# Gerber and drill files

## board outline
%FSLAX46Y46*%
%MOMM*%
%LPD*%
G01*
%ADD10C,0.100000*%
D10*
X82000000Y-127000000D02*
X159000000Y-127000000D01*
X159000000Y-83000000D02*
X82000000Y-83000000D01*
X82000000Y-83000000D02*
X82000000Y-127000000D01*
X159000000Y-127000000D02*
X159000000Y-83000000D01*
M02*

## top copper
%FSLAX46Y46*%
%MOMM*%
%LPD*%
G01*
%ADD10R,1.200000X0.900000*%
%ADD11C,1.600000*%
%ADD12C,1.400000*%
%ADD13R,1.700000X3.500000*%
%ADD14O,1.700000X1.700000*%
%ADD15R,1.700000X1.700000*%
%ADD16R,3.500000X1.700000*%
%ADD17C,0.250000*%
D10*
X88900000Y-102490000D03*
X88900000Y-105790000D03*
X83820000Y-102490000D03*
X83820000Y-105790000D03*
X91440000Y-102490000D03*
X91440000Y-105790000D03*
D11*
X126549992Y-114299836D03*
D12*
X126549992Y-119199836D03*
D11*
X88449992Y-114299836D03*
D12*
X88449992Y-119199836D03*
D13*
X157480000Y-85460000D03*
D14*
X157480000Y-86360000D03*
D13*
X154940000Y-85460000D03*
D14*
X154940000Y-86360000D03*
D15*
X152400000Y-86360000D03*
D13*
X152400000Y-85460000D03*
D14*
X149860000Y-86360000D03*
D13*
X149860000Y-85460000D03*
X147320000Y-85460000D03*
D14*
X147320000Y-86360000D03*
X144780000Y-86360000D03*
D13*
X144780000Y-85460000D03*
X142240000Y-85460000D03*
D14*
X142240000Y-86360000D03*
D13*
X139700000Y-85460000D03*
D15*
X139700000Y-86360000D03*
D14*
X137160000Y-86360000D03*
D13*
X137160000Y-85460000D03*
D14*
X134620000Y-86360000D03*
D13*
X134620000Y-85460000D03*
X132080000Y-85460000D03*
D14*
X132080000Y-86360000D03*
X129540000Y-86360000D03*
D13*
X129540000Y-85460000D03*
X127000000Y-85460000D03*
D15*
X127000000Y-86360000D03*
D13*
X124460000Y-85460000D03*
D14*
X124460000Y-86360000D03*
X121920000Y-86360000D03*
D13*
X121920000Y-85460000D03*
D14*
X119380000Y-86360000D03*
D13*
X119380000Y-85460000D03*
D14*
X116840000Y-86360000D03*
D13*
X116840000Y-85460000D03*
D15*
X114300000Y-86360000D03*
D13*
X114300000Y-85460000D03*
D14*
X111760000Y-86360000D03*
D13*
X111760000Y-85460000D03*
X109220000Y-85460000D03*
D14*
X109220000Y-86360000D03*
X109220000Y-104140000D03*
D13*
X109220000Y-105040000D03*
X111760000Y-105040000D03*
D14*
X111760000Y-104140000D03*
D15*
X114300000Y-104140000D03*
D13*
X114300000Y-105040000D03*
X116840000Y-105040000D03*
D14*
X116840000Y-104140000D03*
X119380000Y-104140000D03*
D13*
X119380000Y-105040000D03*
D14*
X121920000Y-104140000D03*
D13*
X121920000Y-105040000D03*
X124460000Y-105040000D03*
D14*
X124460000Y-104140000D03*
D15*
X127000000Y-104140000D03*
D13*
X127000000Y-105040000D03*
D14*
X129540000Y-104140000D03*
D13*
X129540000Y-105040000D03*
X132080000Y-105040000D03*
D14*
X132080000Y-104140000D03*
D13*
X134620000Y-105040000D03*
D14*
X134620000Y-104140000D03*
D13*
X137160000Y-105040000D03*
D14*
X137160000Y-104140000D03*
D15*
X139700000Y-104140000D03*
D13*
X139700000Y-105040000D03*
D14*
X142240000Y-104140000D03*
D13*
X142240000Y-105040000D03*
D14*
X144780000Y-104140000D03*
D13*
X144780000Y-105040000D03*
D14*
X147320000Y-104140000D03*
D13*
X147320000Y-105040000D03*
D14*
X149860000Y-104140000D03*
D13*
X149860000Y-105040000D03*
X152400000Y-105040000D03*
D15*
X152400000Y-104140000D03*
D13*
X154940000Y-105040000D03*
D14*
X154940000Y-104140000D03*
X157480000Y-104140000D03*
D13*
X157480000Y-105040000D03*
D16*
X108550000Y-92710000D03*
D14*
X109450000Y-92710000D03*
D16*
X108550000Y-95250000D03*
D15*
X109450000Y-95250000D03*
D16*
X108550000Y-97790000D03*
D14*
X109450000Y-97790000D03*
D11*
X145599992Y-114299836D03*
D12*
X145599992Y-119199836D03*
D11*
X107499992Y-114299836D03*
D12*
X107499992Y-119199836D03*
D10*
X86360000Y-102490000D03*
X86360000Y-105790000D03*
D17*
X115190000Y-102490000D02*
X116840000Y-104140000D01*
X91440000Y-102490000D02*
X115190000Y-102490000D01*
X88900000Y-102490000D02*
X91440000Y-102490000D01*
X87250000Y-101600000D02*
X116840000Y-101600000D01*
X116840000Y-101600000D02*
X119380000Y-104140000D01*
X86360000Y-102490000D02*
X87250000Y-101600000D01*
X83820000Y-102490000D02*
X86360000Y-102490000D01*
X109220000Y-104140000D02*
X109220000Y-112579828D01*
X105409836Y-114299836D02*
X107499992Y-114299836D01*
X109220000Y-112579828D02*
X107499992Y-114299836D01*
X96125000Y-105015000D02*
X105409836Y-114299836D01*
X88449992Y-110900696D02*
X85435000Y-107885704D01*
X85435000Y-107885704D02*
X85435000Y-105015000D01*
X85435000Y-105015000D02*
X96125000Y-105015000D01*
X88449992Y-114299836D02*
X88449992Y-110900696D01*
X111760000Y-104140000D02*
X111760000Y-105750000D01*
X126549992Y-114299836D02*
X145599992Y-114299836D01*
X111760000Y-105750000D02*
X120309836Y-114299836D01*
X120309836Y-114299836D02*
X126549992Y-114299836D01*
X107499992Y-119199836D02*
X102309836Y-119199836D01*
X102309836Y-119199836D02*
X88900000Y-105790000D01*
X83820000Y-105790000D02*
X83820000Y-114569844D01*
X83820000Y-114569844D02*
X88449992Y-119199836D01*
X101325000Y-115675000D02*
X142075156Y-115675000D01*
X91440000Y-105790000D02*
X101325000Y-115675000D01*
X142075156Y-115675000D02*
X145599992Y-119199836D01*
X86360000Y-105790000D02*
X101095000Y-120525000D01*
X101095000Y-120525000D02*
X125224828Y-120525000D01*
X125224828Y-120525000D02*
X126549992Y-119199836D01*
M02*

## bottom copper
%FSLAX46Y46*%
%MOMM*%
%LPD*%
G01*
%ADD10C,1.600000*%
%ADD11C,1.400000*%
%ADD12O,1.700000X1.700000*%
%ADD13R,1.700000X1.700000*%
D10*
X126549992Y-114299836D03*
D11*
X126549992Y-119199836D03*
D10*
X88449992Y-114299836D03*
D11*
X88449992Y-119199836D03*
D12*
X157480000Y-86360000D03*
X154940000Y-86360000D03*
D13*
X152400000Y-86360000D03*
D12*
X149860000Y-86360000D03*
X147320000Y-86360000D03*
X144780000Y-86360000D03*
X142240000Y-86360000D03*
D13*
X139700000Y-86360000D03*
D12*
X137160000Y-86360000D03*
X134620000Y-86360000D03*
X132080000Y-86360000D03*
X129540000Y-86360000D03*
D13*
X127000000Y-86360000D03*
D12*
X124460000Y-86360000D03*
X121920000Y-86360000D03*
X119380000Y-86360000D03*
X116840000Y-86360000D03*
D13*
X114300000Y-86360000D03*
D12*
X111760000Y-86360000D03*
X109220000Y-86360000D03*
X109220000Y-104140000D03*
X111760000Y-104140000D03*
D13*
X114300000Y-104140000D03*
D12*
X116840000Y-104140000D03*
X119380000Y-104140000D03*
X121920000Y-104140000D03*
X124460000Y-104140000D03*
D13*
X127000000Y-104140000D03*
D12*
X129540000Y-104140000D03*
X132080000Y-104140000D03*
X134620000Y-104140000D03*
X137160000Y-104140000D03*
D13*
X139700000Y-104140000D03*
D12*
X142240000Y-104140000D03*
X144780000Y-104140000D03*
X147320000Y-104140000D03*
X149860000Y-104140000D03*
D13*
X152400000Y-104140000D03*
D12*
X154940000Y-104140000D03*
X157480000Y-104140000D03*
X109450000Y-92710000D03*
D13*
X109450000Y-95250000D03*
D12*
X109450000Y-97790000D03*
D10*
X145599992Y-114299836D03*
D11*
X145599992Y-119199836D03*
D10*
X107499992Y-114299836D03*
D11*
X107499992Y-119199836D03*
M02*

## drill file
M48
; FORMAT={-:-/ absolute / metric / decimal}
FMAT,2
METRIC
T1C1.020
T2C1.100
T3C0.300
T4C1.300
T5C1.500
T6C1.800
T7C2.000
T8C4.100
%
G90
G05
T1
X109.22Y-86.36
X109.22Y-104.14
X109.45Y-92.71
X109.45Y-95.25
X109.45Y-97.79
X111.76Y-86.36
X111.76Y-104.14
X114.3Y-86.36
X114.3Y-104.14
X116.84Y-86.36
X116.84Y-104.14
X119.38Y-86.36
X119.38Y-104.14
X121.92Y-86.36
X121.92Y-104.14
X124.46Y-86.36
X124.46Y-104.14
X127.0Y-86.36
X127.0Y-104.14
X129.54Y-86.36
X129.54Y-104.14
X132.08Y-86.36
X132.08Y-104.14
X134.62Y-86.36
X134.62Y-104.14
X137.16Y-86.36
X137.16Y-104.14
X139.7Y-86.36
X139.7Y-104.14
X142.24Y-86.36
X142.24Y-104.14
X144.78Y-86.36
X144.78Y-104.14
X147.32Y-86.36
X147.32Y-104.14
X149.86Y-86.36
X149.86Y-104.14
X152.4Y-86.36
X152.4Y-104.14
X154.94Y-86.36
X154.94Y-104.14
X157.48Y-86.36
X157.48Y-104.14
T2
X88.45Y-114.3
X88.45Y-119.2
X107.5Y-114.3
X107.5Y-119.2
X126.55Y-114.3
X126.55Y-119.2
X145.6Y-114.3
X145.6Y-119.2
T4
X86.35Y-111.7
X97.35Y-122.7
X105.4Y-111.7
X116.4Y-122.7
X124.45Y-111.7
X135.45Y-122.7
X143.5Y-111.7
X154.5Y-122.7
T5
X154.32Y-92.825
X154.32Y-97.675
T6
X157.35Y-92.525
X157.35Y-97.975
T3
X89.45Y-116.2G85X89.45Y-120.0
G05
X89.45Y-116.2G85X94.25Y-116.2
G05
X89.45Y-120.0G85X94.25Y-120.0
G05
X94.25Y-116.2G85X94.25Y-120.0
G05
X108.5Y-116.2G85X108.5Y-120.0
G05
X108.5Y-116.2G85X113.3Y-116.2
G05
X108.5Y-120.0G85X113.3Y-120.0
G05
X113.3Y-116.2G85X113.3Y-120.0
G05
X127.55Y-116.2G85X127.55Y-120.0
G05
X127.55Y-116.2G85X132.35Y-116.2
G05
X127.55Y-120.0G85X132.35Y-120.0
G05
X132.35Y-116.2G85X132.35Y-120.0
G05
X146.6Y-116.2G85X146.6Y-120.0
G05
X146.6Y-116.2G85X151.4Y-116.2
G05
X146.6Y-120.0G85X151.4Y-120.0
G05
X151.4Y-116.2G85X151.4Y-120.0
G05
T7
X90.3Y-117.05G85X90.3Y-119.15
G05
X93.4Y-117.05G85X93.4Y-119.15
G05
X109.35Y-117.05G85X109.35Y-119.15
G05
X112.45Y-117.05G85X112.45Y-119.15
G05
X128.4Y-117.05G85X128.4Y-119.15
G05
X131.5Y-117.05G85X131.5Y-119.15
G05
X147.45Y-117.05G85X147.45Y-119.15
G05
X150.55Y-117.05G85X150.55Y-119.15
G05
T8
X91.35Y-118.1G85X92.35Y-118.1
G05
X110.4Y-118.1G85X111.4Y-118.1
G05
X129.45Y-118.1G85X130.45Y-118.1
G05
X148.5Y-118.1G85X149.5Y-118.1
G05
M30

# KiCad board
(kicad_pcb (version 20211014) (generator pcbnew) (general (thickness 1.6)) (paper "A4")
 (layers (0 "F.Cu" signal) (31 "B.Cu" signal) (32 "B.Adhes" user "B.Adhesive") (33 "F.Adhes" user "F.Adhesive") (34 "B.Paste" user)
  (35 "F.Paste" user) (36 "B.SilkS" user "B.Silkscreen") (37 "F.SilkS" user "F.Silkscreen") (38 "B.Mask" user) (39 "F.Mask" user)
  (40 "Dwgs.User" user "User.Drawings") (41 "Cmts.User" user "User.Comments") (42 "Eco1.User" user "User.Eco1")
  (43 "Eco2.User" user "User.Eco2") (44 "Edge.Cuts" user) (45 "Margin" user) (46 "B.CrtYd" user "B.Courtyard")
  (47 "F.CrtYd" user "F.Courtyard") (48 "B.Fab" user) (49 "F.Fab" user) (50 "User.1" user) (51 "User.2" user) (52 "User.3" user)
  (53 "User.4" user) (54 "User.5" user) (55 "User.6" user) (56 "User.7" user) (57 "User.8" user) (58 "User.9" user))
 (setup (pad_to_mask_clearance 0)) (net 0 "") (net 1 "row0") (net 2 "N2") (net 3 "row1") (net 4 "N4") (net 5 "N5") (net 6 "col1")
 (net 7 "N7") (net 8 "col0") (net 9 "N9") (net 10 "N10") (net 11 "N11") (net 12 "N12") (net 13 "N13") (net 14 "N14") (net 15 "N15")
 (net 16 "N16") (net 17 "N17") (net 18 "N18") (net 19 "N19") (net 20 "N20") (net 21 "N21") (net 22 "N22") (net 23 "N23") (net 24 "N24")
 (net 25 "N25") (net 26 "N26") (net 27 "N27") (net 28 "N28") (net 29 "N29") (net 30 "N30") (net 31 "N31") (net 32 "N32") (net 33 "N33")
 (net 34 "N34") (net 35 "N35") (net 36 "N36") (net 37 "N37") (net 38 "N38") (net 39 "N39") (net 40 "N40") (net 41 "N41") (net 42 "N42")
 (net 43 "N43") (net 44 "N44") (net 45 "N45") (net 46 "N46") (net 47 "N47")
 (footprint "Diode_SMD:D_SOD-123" (layer "F.Cu") (at 88.9 104.14 -90)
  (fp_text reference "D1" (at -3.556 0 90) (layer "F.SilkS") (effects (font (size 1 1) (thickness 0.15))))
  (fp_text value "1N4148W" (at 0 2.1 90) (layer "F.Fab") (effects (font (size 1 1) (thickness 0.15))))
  (pad "1" smd rect (at -1.65 0 270) (size 0.9 1.2) (layers "F.Cu" "F.Paste" "F.Mask") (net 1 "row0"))
  (pad "2" smd rect (at 1.65 0 270) (size 0.9 1.2) (layers "F.Cu" "F.Paste" "F.Mask") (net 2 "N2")))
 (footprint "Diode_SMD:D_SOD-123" (layer "F.Cu") (at 83.82 104.14 -90)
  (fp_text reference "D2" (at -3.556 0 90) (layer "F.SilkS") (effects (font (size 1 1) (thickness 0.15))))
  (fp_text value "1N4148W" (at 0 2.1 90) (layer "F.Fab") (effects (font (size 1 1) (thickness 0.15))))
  (pad "1" smd rect (at -1.65 0 270) (size 0.9 1.2) (layers "F.Cu" "F.Paste" "F.Mask") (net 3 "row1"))
  (pad "2" smd rect (at 1.65 0 270) (size 0.9 1.2) (layers "F.Cu" "F.Paste" "F.Mask") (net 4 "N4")))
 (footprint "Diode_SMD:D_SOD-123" (layer "F.Cu") (at 91.44 104.14 -90)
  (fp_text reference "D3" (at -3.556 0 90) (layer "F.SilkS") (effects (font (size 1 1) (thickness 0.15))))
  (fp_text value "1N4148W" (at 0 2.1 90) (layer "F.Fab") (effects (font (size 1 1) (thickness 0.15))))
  (pad "1" smd rect (at -1.65 0 270) (size 0.9 1.2) (layers "F.Cu" "F.Paste" "F.Mask") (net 1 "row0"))
  (pad "2" smd rect (at 1.65 0 270) (size 0.9 1.2) (layers "F.Cu" "F.Paste" "F.Mask") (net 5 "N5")))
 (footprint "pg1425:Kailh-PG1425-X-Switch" (layer "F.Cu") (at 133.35 114.3)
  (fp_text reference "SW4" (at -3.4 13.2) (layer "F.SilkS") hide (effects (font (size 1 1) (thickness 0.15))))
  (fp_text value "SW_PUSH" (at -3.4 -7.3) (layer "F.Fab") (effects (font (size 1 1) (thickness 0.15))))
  (pad "" np_thru_hole oval locked (at -3.4 3.8) (size 5.1 4.1) (drill oval 5.1 4.1) (layers *.Cu *.Mask))
  (pad "" np_thru_hole oval locked (at -1.85 3.8) (size 2 4.1) (drill oval 2 4.1) (layers *.Cu *.Mask))
  (pad "" np_thru_hole oval locked (at -5.8 3.8) (size 0.3 4.1) (drill oval 0.3 4.1) (layers *.Cu *.Mask))
  (pad "" np_thru_hole oval locked (at -3.4 1.9) (size 5.1 0.3) (drill oval 5.1 0.3) (layers *.Cu *.Mask))
  (pad "" np_thru_hole circle locked (at -8.900008 -2.600164 180) (size 1.3 1.3) (drill 1.3) (layers *.Cu *.Mask))
  (pad "" np_thru_hole oval locked (at -3.4 5.7) (size 5.1 0.3) (drill oval 5.1 0.3) (layers *.Cu *.Mask))
  (pad "" np_thru_hole oval locked (at -4.95 3.8) (size 2 4.1) (drill oval 2 4.1) (layers *.Cu *.Mask))
  (pad "" np_thru_hole oval locked (at -1 3.8) (size 0.3 4.1) (drill oval 0.3 4.1) (layers *.Cu *.Mask))
  (pad "" np_thru_hole circle locked (at 2.099992 8.399836 180) (size 1.3 1.3) (drill 1.3) (layers *.Cu *.Mask))
  (pad "1" thru_hole circle locked (at -6.800008 -0.000164 180) (size 1.6 1.6) (drill 1.1) (layers *.Cu *.Mask) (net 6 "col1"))
  (pad "2" thru_hole circle locked (at -6.800008 4.899836 180) (size 1.4 1.4) (drill 1.1) (layers *.Cu *.Mask) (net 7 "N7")))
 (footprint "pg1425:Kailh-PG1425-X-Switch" (layer "F.Cu") (at 95.25 114.3)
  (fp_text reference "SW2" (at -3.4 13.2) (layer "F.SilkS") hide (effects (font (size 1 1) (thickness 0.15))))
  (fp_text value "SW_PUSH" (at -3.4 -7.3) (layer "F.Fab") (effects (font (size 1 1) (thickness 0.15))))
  (pad "" np_thru_hole oval locked (at -4.95 3.8) (size 2 4.1) (drill oval 2 4.1) (layers *.Cu *.Mask))
  (pad "" np_thru_hole oval locked (at -5.8 3.8) (size 0.3 4.1) (drill oval 0.3 4.1) (layers *.Cu *.Mask))
  (pad "" np_thru_hole oval locked (at -1 3.8) (size 0.3 4.1) (drill oval 0.3 4.1) (layers *.Cu *.Mask))
  (pad "" np_thru_hole oval locked (at -1.85 3.8) (size 2 4.1) (drill oval 2 4.1) (layers *.Cu *.Mask))
  (pad "" np_thru_hole circle locked (at -8.900008 -2.600164 180) (size 1.3 1.3) (drill 1.3) (layers *.Cu *.Mask))
  (pad "" np_thru_hole oval locked (at -3.4 3.8) (size 5.1 4.1) (drill oval 5.1 4.1) (layers *.Cu *.Mask))
  (pad "" np_thru_hole oval locked (at -3.4 5.7) (size 5.1 0.3) (drill oval 5.1 0.3) (layers *.Cu *.Mask))
  (pad "" np_thru_hole oval locked (at -3.4 1.9) (size 5.1 0.3) (drill oval 5.1 0.3) (layers *.Cu *.Mask))
  (pad "" np_thru_hole circle locked (at 2.099992 8.399836 180) (size 1.3 1.3) (drill 1.3) (layers *.Cu *.Mask))
  (pad "1" thru_hole circle locked (at -6.800008 -0.000164 180) (size 1.6 1.6) (drill 1.1) (layers *.Cu *.Mask) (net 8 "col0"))
  (pad "2" thru_hole circle locked (at -6.800008 4.899836 180) (size 1.4 1.4) (drill 1.1) (layers *.Cu *.Mask) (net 4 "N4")))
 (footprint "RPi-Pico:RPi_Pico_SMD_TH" (layer "F.Cu") (at 133.35 95.25 -90)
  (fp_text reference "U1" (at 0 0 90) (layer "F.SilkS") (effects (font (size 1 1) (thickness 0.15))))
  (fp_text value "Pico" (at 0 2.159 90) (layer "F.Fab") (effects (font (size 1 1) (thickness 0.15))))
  (pad "" np_thru_hole oval (at 2.725 -24 270) (size 1.8 1.8) (drill 1.8) (layers *.Cu *.Mask))
  (pad "" np_thru_hole oval (at -2.425 -20.97 270) (size 1.5 1.5) (drill 1.5) (layers *.Cu *.Mask))
  (pad "" np_thru_hole oval (at -2.725 -24 270) (size 1.8 1.8) (drill 1.8) (layers *.Cu *.Mask))
  (pad "" np_thru_hole oval (at 2.425 -20.97 270) (size 1.5 1.5) (drill 1.5) (layers *.Cu *.Mask))
  (pad "1" smd rect (at -8.89 -24.13 270) (size 3.5 1.7) (drill (offset -0.9 0)) (layers "F.Cu" "F.Mask") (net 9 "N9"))
  (pad "1" thru_hole oval (at -8.89 -24.13 270) (size 1.7 1.7) (drill 1.02) (layers *.Cu *.Mask) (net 9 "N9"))
  (pad "2" smd rect (at -8.89 -21.59 270) (size 3.5 1.7) (drill (offset -0.9 0)) (layers "F.Cu" "F.Mask") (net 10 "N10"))
  (pad "2" thru_hole oval (at -8.89 -21.59 270) (size 1.7 1.7) (drill 1.02) (layers *.Cu *.Mask) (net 10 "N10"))
  (pad "3" thru_hole rect (at -8.89 -19.05 270) (size 1.7 1.7) (drill 1.02) (layers *.Cu *.Mask) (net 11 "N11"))
  (pad "3" smd rect (at -8.89 -19.05 270) (size 3.5 1.7) (drill (offset -0.9 0)) (layers "F.Cu" "F.Mask") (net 11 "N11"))
  (pad "4" thru_hole oval (at -8.89 -16.51 270) (size 1.7 1.7) (drill 1.02) (layers *.Cu *.Mask) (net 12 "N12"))
  (pad "4" smd rect (at -8.89 -16.51 270) (size 3.5 1.7) (drill (offset -0.9 0)) (layers "F.Cu" "F.Mask") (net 12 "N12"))
  (pad "5" smd rect (at -8.89 -13.97 270) (size 3.5 1.7) (drill (offset -0.9 0)) (layers "F.Cu" "F.Mask") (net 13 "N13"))
  (pad "5" thru_hole oval (at -8.89 -13.97 270) (size 1.7 1.7) (drill 1.02) (layers *.Cu *.Mask) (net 13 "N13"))
  (pad "6" thru_hole oval (at -8.89 -11.43 270) (size 1.7 1.7) (drill 1.02) (layers *.Cu *.Mask) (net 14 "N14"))
  (pad "6" smd rect (at -8.89 -11.43 270) (size 3.5 1.7) (drill (offset -0.9 0)) (layers "F.Cu" "F.Mask") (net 14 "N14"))
  (pad "7" smd rect (at -8.89 -8.89 270) (size 3.5 1.7) (drill (offset -0.9 0)) (layers "F.Cu" "F.Mask") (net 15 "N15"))
  (pad "7" thru_hole oval (at -8.89 -8.89 270) (size 1.7 1.7) (drill 1.02) (layers *.Cu *.Mask) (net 15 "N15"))
  (pad "8" smd rect (at -8.89 -6.35 270) (size 3.5 1.7) (drill (offset -0.9 0)) (layers "F.Cu" "F.Mask") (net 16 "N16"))
  (pad "8" thru_hole rect (at -8.89 -6.35 270) (size 1.7 1.7) (drill 1.02) (layers *.Cu *.Mask) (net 16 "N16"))
  (pad "9" thru_hole oval (at -8.89 -3.81 270) (size 1.7 1.7) (drill 1.02) (layers *.Cu *.Mask) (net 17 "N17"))
  (pad "9" smd rect (at -8.89 -3.81 270) (size 3.5 1.7) (drill (offset -0.9 0)) (layers "F.Cu" "F.Mask") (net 17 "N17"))
  (pad "10" thru_hole oval (at -8.89 -1.27 270) (size 1.7 1.7) (drill 1.02) (layers *.Cu *.Mask) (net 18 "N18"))
  (pad "10" smd rect (at -8.89 -1.27 270) (size 3.5 1.7) (drill (offset -0.9 0)) (layers "F.Cu" "F.Mask") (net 18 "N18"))
  (pad "11" smd rect (at -8.89 1.27 270) (size 3.5 1.7) (drill (offset -0.9 0)) (layers "F.Cu" "F.Mask") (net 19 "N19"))
  (pad "11" thru_hole oval (at -8.89 1.27 270) (size 1.7 1.7) (drill 1.02) (layers *.Cu *.Mask) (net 19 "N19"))
  (pad "12" thru_hole oval (at -8.89 3.81 270) (size 1.7 1.7) (drill 1.02) (layers *.Cu *.Mask) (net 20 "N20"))
  (pad "12" smd rect (at -8.89 3.81 270) (size 3.5 1.7) (drill (offset -0.9 0)) (layers "F.Cu" "F.Mask") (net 20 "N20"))
  (pad "13" smd rect (at -8.89 6.35 270) (size 3.5 1.7) (drill (offset -0.9 0)) (layers "F.Cu" "F.Mask") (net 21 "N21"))
  (pad "13" thru_hole rect (at -8.89 6.35 270) (size 1.7 1.7) (drill 1.02) (layers *.Cu *.Mask) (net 21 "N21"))
  (pad "14" smd rect (at -8.89 8.89 270) (size 3.5 1.7) (drill (offset -0.9 0)) (layers "F.Cu" "F.Mask") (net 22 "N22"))
  (pad "14" thru_hole oval (at -8.89 8.89 270) (size 1.7 1.7) (drill 1.02) (layers *.Cu *.Mask) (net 22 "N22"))
  (pad "15" thru_hole oval (at -8.89 11.43 270) (size 1.7 1.7) (drill 1.02) (layers *.Cu *.Mask) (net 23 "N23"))
  (pad "15" smd rect (at -8.89 11.43 270) (size 3.5 1.7) (drill (offset -0.9 0)) (layers "F.Cu" "F.Mask") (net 23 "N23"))
  (pad "16" thru_hole oval (at -8.89 13.97 270) (size 1.7 1.7) (drill 1.02) (layers *.Cu *.Mask) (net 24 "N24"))
  (pad "16" smd rect (at -8.89 13.97 270) (size 3.5 1.7) (drill (offset -0.9 0)) (layers "F.Cu" "F.Mask") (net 24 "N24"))
  (pad "17" thru_hole oval (at -8.89 16.51 270) (size 1.7 1.7) (drill 1.02) (layers *.Cu *.Mask) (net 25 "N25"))
  (pad "17" smd rect (at -8.89 16.51 270) (size 3.5 1.7) (drill (offset -0.9 0)) (layers "F.Cu" "F.Mask") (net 25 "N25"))
  (pad "18" thru_hole rect (at -8.89 19.05 270) (size 1.7 1.7) (drill 1.02) (layers *.Cu *.Mask) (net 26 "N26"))
  (pad "18" smd rect (at -8.89 19.05 270) (size 3.5 1.7) (drill (offset -0.9 0)) (layers "F.Cu" "F.Mask") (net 26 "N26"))
  (pad "19" thru_hole oval (at -8.89 21.59 270) (size 1.7 1.7) (drill 1.02) (layers *.Cu *.Mask) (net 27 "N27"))
  (pad "19" smd rect (at -8.89 21.59 270) (size 3.5 1.7) (drill (offset -0.9 0)) (layers "F.Cu" "F.Mask") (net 27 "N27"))
  (pad "20" smd rect (at -8.89 24.13 270) (size 3.5 1.7) (drill (offset -0.9 0)) (layers "F.Cu" "F.Mask") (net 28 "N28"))
  (pad "20" thru_hole oval (at -8.89 24.13 270) (size 1.7 1.7) (drill 1.02) (layers *.Cu *.Mask) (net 28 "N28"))
  (pad "21" thru_hole oval (at 8.89 24.13 270) (size 1.7 1.7) (drill 1.02) (layers *.Cu *.Mask) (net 8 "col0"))
  (pad "21" smd rect (at 8.89 24.13 270) (size 3.5 1.7) (drill (offset 0.9 0)) (layers "F.Cu" "F.Mask") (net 8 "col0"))
  (pad "22" smd rect (at 8.89 21.59 270) (size 3.5 1.7) (drill (offset 0.9 0)) (layers "F.Cu" "F.Mask") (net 6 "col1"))
  (pad "22" thru_hole oval (at 8.89 21.59 270) (size 1.7 1.7) (drill 1.02) (layers *.Cu *.Mask) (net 6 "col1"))
  (pad "23" thru_hole rect (at 8.89 19.05 270) (size 1.7 1.7) (drill 1.02) (layers *.Cu *.Mask) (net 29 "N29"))
  (pad "23" smd rect (at 8.89 19.05 270) (size 3.5 1.7) (drill (offset 0.9 0)) (layers "F.Cu" "F.Mask") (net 29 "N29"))
  (pad "24" smd rect (at 8.89 16.51 270) (size 3.5 1.7) (drill (offset 0.9 0)) (layers "F.Cu" "F.Mask") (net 1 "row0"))
  (pad "24" thru_hole oval (at 8.89 16.51 270) (size 1.7 1.7) (drill 1.02) (layers *.Cu *.Mask) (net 1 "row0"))
  (pad "25" thru_hole oval (at 8.89 13.97 270) (size 1.7 1.7) (drill 1.02) (layers *.Cu *.Mask) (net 3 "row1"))
  (pad "25" smd rect (at 8.89 13.97 270) (size 3.5 1.7) (drill (offset 0.9 0)) (layers "F.Cu" "F.Mask") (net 3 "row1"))
  (pad "26" thru_hole oval (at 8.89 11.43 270) (size 1.7 1.7) (drill 1.02) (layers *.Cu *.Mask) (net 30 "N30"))
  (pad "26" smd rect (at 8.89 11.43 270) (size 3.5 1.7) (drill (offset 0.9 0)) (layers "F.Cu" "F.Mask") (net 30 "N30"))
  (pad "27" smd rect (at 8.89 8.89 270) (size 3.5 1.7) (drill (offset 0.9 0)) (layers "F.Cu" "F.Mask") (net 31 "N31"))
  (pad "27" thru_hole oval (at 8.89 8.89 270) (size 1.7 1.7) (drill 1.02) (layers *.Cu *.Mask) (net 31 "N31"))
  (pad "28" thru_hole rect (at 8.89 6.35 270) (size 1.7 1.7) (drill 1.02) (layers *.Cu *.Mask) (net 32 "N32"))
  (pad "28" smd rect (at 8.89 6.35 270) (size 3.5 1.7) (drill (offset 0.9 0)) (layers "F.Cu" "F.Mask") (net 32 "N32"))
  (pad "29" thru_hole oval (at 8.89 3.81 270) (size 1.7 1.7) (drill 1.02) (layers *.Cu *.Mask) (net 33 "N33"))
  (pad "29" smd rect (at 8.89 3.81 270) (size 3.5 1.7) (drill (offset 0.9 0)) (layers "F.Cu" "F.Mask") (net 33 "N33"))
  (pad "30" smd rect (at 8.89 1.27 270) (size 3.5 1.7) (drill (offset 0.9 0)) (layers "F.Cu" "F.Mask") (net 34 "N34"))
  (pad "30" thru_hole oval (at 8.89 1.27 270) (size 1.7 1.7) (drill 1.02) (layers *.Cu *.Mask) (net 34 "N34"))
  (pad "31" smd rect (at 8.89 -1.27 270) (size 3.5 1.7) (drill (offset 0.9 0)) (layers "F.Cu" "F.Mask") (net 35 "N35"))
  (pad "31" thru_hole oval (at 8.89 -1.27 270) (size 1.7 1.7) (drill 1.02) (layers *.Cu *.Mask) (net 35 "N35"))
  (pad "32" smd rect (at 8.89 -3.81 270) (size 3.5 1.7) (drill (offset 0.9 0)) (layers "F.Cu" "F.Mask") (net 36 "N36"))
  (pad "32" thru_hole oval (at 8.89 -3.81 270) (size 1.7 1.7) (drill 1.02) (layers *.Cu *.Mask) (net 36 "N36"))
  (pad "33" thru_hole rect (at 8.89 -6.35 270) (size 1.7 1.7) (drill 1.02) (layers *.Cu *.Mask) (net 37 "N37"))
  (pad "33" smd rect (at 8.89 -6.35 270) (size 3.5 1.7) (drill (offset 0.9 0)) (layers "F.Cu" "F.Mask") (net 37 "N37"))
  (pad "34" thru_hole oval (at 8.89 -8.89 270) (size 1.7 1.7) (drill 1.02) (layers *.Cu *.Mask) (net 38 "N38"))
  (pad "34" smd rect (at 8.89 -8.89 270) (size 3.5 1.7) (drill (offset 0.9 0)) (layers "F.Cu" "F.Mask") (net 38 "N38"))
  (pad "35" thru_hole oval (at 8.89 -11.43 270) (size 1.7 1.7) (drill 1.02) (layers *.Cu *.Mask) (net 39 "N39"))
  (pad "35" smd rect (at 8.89 -11.43 270) (size 3.5 1.7) (drill (offset 0.9 0)) (layers "F.Cu" "F.Mask") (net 39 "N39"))
  (pad "36" thru_hole oval (at 8.89 -13.97 270) (size 1.7 1.7) (drill 1.02) (layers *.Cu *.Mask) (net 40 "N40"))
  (pad "36" smd rect (at 8.89 -13.97 270) (size 3.5 1.7) (drill (offset 0.9 0)) (layers "F.Cu" "F.Mask") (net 40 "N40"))
  (pad "37" thru_hole oval (at 8.89 -16.51 270) (size 1.7 1.7) (drill 1.02) (layers *.Cu *.Mask) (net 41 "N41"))
  (pad "37" smd rect (at 8.89 -16.51 270) (size 3.5 1.7) (drill (offset 0.9 0)) (layers "F.Cu" "F.Mask") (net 41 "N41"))
  (pad "38" smd rect (at 8.89 -19.05 270) (size 3.5 1.7) (drill (offset 0.9 0)) (layers "F.Cu" "F.Mask") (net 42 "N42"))
  (pad "38" thru_hole rect (at 8.89 -19.05 270) (size 1.7 1.7) (drill 1.02) (layers *.Cu *.Mask) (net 42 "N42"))
  (pad "39" smd rect (at 8.89 -21.59 270) (size 3.5 1.7) (drill (offset 0.9 0)) (layers "F.Cu" "F.Mask") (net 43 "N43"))
  (pad "39" thru_hole oval (at 8.89 -21.59 270) (size 1.7 1.7) (drill 1.02) (layers *.Cu *.Mask) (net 43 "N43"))
  (pad "40" thru_hole oval (at 8.89 -24.13 270) (size 1.7 1.7) (drill 1.02) (layers *.Cu *.Mask) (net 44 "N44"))
  (pad "40" smd rect (at 8.89 -24.13 270) (size 3.5 1.7) (drill (offset 0.9 0)) (layers "F.Cu" "F.Mask") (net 44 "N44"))
  (pad "41" smd rect (at -2.54 23.9) (size 3.5 1.7) (drill (offset -0.9 0)) (layers "F.Cu" "F.Mask") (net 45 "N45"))
  (pad "41" thru_hole oval (at -2.54 23.9 270) (size 1.7 1.7) (drill 1.02) (layers *.Cu *.Mask) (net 45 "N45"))
  (pad "42" smd rect (at 0 23.9) (size 3.5 1.7) (drill (offset -0.9 0)) (layers "F.Cu" "F.Mask") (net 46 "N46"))
  (pad "42" thru_hole rect (at 0 23.9 270) (size 1.7 1.7) (drill 1.02) (layers *.Cu *.Mask) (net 46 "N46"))
  (pad "43" smd rect (at 2.54 23.9) (size 3.5 1.7) (drill (offset -0.9 0)) (layers "F.Cu" "F.Mask") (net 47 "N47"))
  (pad "43" thru_hole oval (at 2.54 23.9 270) (size 1.7 1.7) (drill 1.02) (layers *.Cu *.Mask) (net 47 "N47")))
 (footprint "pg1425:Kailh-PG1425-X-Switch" (layer "F.Cu") (at 152.4 114.3)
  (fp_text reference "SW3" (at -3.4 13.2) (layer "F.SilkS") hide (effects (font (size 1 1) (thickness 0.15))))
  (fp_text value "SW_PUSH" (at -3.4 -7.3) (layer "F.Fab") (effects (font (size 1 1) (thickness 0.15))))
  (pad "" np_thru_hole oval locked (at -1.85 3.8) (size 2 4.1) (drill oval 2 4.1) (layers *.Cu *.Mask))
  (pad "" np_thru_hole circle locked (at 2.099992 8.399836 180) (size 1.3 1.3) (drill 1.3) (layers *.Cu *.Mask))
  (pad "" np_thru_hole circle locked (at -8.900008 -2.600164 180) (size 1.3 1.3) (drill 1.3) (layers *.Cu *.Mask))
  (pad "" np_thru_hole oval locked (at -3.4 1.9) (size 5.1 0.3) (drill oval 5.1 0.3) (layers *.Cu *.Mask))
  (pad "" np_thru_hole oval locked (at -1 3.8) (size 0.3 4.1) (drill oval 0.3 4.1) (layers *.Cu *.Mask))
  (pad "" np_thru_hole oval locked (at -3.4 3.8) (size 5.1 4.1) (drill oval 5.1 4.1) (layers *.Cu *.Mask))
  (pad "" np_thru_hole oval locked (at -3.4 5.7) (size 5.1 0.3) (drill oval 5.1 0.3) (layers *.Cu *.Mask))
  (pad "" np_thru_hole oval locked (at -5.8 3.8) (size 0.3 4.1) (drill oval 0.3 4.1) (layers *.Cu *.Mask))
  (pad "" np_thru_hole oval locked (at -4.95 3.8) (size 2 4.1) (drill oval 2 4.1) (layers *.Cu *.Mask))
  (pad "1" thru_hole circle locked (at -6.800008 -0.000164 180) (size 1.6 1.6) (drill 1.1) (layers *.Cu *.Mask) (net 6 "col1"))
  (pad "2" thru_hole circle locked (at -6.800008 4.899836 180) (size 1.4 1.4) (drill 1.1) (layers *.Cu *.Mask) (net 5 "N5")))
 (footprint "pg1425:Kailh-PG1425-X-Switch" (layer "F.Cu") (at 114.3 114.3)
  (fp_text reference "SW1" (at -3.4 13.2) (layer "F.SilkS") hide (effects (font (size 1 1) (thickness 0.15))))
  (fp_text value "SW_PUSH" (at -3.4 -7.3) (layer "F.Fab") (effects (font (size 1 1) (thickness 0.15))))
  (pad "" np_thru_hole oval locked (at -3.4 3.8) (size 5.1 4.1) (drill oval 5.1 4.1) (layers *.Cu *.Mask))
  (pad "" np_thru_hole oval locked (at -5.8 3.8) (size 0.3 4.1) (drill oval 0.3 4.1) (layers *.Cu *.Mask))
  (pad "" np_thru_hole oval locked (at -1 3.8) (size 0.3 4.1) (drill oval 0.3 4.1) (layers *.Cu *.Mask))
  (pad "" np_thru_hole circle locked (at -8.900008 -2.600164 180) (size 1.3 1.3) (drill 1.3) (layers *.Cu *.Mask))
  (pad "" np_thru_hole oval locked (at -3.4 1.9) (size 5.1 0.3) (drill oval 5.1 0.3) (layers *.Cu *.Mask))
  (pad "" np_thru_hole oval locked (at -3.4 5.7) (size 5.1 0.3) (drill oval 5.1 0.3) (layers *.Cu *.Mask))
  (pad "" np_thru_hole oval locked (at -1.85 3.8) (size 2 4.1) (drill oval 2 4.1) (layers *.Cu *.Mask))
  (pad "" np_thru_hole circle locked (at 2.099992 8.399836 180) (size 1.3 1.3) (drill 1.3) (layers *.Cu *.Mask))
  (pad "" np_thru_hole oval locked (at -4.95 3.8) (size 2 4.1) (drill oval 2 4.1) (layers *.Cu *.Mask))
  (pad "1" thru_hole circle locked (at -6.800008 -0.000164 180) (size 1.6 1.6) (drill 1.1) (layers *.Cu *.Mask) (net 8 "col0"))
  (pad "2" thru_hole circle locked (at -6.800008 4.899836 180) (size 1.4 1.4) (drill 1.1) (layers *.Cu *.Mask) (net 2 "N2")))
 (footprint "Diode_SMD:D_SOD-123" (layer "F.Cu") (at 86.36 104.14 -90)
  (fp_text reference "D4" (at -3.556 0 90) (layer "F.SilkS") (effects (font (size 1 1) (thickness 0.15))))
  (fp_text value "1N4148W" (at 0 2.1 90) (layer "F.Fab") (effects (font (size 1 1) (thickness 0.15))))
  (pad "1" smd rect (at -1.65 0 270) (size 0.9 1.2) (layers "F.Cu" "F.Paste" "F.Mask") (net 3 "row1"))
  (pad "2" smd rect (at 1.65 0 270) (size 0.9 1.2) (layers "F.Cu" "F.Paste" "F.Mask") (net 7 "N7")))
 (gr_line (start 82 127) (end 159 127) (layer "Edge.Cuts") (width 0.1))
 (gr_line (start 159 83) (end 82 83) (layer "Edge.Cuts") (width 0.1))
 (gr_line (start 82 83) (end 82 127) (layer "Edge.Cuts") (width 0.1))
 (gr_line (start 159 127) (end 159 83) (layer "Edge.Cuts") (width 0.1))
 (segment (start 115.19 102.49) (end 116.84 104.14) (width 0.25) (layer "F.Cu") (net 1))
 (segment (start 91.44 102.49) (end 115.19 102.49) (width 0.25) (layer "F.Cu") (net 1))
 (segment (start 88.9 102.49) (end 91.44 102.49) (width 0.25) (layer "F.Cu") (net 1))
 (segment (start 87.25 101.6) (end 116.84 101.6) (width 0.25) (layer "F.Cu") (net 3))
 (segment (start 116.84 101.6) (end 119.38 104.14) (width 0.25) (layer "F.Cu") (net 3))
 (segment (start 86.36 102.49) (end 87.25 101.6) (width 0.25) (layer "F.Cu") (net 3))
 (segment (start 83.82 102.49) (end 86.36 102.49) (width 0.25) (layer "F.Cu") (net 3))
 (segment (start 109.22 104.14) (end 109.22 112.579828) (width 0.25) (layer "F.Cu") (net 8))
 (segment (start 105.409836 114.299836) (end 107.499992 114.299836) (width 0.25) (layer "F.Cu") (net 8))
 (segment (start 109.22 112.579828) (end 107.499992 114.299836) (width 0.25) (layer "F.Cu") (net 8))
 (segment (start 96.125 105.015) (end 105.409836 114.299836) (width 0.25) (layer "F.Cu") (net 8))
 (segment (start 88.449992 110.900696) (end 85.435 107.885704) (width 0.25) (layer "F.Cu") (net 8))
 (segment (start 85.435 107.885704) (end 85.435 105.015) (width 0.25) (layer "F.Cu") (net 8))
 (segment (start 85.435 105.015) (end 96.125 105.015) (width 0.25) (layer "F.Cu") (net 8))
 (segment (start 88.449992 114.299836) (end 88.449992 110.900696) (width 0.25) (layer "F.Cu") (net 8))
 (segment (start 111.76 104.14) (end 111.76 105.75) (width 0.25) (layer "F.Cu") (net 6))
 (segment (start 126.549992 114.299836) (end 145.599992 114.299836) (width 0.25) (layer "F.Cu") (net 6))
 (segment (start 111.76 105.75) (end 120.309836 114.299836) (width 0.25) (layer "F.Cu") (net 6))
 (segment (start 120.309836 114.299836) (end 126.549992 114.299836) (width 0.25) (layer "F.Cu") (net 6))
 (segment (start 107.499992 119.199836) (end 102.309836 119.199836) (width 0.25) (layer "F.Cu") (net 2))
 (segment (start 102.309836 119.199836) (end 88.9 105.79) (width 0.25) (layer "F.Cu") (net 2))
 (segment (start 83.82 105.79) (end 83.82 114.569844) (width 0.25) (layer "F.Cu") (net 4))
 (segment (start 83.82 114.569844) (end 88.449992 119.199836) (width 0.25) (layer "F.Cu") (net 4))
 (segment (start 101.325 115.675) (end 142.075156 115.675) (width 0.25) (layer "F.Cu") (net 5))
 (segment (start 91.44 105.79) (end 101.325 115.675) (width 0.25) (layer "F.Cu") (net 5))
 (segment (start 142.075156 115.675) (end 145.599992 119.199836) (width 0.25) (layer "F.Cu") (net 5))
 (segment (start 86.36 105.79) (end 101.095 120.525) (width 0.25) (layer "F.Cu") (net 7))
 (segment (start 101.095 120.525) (end 125.224828 120.525) (width 0.25) (layer "F.Cu") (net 7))
 (segment (start 125.224828 120.525) (end 126.549992 119.199836) (width 0.25) (layer "F.Cu") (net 7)))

